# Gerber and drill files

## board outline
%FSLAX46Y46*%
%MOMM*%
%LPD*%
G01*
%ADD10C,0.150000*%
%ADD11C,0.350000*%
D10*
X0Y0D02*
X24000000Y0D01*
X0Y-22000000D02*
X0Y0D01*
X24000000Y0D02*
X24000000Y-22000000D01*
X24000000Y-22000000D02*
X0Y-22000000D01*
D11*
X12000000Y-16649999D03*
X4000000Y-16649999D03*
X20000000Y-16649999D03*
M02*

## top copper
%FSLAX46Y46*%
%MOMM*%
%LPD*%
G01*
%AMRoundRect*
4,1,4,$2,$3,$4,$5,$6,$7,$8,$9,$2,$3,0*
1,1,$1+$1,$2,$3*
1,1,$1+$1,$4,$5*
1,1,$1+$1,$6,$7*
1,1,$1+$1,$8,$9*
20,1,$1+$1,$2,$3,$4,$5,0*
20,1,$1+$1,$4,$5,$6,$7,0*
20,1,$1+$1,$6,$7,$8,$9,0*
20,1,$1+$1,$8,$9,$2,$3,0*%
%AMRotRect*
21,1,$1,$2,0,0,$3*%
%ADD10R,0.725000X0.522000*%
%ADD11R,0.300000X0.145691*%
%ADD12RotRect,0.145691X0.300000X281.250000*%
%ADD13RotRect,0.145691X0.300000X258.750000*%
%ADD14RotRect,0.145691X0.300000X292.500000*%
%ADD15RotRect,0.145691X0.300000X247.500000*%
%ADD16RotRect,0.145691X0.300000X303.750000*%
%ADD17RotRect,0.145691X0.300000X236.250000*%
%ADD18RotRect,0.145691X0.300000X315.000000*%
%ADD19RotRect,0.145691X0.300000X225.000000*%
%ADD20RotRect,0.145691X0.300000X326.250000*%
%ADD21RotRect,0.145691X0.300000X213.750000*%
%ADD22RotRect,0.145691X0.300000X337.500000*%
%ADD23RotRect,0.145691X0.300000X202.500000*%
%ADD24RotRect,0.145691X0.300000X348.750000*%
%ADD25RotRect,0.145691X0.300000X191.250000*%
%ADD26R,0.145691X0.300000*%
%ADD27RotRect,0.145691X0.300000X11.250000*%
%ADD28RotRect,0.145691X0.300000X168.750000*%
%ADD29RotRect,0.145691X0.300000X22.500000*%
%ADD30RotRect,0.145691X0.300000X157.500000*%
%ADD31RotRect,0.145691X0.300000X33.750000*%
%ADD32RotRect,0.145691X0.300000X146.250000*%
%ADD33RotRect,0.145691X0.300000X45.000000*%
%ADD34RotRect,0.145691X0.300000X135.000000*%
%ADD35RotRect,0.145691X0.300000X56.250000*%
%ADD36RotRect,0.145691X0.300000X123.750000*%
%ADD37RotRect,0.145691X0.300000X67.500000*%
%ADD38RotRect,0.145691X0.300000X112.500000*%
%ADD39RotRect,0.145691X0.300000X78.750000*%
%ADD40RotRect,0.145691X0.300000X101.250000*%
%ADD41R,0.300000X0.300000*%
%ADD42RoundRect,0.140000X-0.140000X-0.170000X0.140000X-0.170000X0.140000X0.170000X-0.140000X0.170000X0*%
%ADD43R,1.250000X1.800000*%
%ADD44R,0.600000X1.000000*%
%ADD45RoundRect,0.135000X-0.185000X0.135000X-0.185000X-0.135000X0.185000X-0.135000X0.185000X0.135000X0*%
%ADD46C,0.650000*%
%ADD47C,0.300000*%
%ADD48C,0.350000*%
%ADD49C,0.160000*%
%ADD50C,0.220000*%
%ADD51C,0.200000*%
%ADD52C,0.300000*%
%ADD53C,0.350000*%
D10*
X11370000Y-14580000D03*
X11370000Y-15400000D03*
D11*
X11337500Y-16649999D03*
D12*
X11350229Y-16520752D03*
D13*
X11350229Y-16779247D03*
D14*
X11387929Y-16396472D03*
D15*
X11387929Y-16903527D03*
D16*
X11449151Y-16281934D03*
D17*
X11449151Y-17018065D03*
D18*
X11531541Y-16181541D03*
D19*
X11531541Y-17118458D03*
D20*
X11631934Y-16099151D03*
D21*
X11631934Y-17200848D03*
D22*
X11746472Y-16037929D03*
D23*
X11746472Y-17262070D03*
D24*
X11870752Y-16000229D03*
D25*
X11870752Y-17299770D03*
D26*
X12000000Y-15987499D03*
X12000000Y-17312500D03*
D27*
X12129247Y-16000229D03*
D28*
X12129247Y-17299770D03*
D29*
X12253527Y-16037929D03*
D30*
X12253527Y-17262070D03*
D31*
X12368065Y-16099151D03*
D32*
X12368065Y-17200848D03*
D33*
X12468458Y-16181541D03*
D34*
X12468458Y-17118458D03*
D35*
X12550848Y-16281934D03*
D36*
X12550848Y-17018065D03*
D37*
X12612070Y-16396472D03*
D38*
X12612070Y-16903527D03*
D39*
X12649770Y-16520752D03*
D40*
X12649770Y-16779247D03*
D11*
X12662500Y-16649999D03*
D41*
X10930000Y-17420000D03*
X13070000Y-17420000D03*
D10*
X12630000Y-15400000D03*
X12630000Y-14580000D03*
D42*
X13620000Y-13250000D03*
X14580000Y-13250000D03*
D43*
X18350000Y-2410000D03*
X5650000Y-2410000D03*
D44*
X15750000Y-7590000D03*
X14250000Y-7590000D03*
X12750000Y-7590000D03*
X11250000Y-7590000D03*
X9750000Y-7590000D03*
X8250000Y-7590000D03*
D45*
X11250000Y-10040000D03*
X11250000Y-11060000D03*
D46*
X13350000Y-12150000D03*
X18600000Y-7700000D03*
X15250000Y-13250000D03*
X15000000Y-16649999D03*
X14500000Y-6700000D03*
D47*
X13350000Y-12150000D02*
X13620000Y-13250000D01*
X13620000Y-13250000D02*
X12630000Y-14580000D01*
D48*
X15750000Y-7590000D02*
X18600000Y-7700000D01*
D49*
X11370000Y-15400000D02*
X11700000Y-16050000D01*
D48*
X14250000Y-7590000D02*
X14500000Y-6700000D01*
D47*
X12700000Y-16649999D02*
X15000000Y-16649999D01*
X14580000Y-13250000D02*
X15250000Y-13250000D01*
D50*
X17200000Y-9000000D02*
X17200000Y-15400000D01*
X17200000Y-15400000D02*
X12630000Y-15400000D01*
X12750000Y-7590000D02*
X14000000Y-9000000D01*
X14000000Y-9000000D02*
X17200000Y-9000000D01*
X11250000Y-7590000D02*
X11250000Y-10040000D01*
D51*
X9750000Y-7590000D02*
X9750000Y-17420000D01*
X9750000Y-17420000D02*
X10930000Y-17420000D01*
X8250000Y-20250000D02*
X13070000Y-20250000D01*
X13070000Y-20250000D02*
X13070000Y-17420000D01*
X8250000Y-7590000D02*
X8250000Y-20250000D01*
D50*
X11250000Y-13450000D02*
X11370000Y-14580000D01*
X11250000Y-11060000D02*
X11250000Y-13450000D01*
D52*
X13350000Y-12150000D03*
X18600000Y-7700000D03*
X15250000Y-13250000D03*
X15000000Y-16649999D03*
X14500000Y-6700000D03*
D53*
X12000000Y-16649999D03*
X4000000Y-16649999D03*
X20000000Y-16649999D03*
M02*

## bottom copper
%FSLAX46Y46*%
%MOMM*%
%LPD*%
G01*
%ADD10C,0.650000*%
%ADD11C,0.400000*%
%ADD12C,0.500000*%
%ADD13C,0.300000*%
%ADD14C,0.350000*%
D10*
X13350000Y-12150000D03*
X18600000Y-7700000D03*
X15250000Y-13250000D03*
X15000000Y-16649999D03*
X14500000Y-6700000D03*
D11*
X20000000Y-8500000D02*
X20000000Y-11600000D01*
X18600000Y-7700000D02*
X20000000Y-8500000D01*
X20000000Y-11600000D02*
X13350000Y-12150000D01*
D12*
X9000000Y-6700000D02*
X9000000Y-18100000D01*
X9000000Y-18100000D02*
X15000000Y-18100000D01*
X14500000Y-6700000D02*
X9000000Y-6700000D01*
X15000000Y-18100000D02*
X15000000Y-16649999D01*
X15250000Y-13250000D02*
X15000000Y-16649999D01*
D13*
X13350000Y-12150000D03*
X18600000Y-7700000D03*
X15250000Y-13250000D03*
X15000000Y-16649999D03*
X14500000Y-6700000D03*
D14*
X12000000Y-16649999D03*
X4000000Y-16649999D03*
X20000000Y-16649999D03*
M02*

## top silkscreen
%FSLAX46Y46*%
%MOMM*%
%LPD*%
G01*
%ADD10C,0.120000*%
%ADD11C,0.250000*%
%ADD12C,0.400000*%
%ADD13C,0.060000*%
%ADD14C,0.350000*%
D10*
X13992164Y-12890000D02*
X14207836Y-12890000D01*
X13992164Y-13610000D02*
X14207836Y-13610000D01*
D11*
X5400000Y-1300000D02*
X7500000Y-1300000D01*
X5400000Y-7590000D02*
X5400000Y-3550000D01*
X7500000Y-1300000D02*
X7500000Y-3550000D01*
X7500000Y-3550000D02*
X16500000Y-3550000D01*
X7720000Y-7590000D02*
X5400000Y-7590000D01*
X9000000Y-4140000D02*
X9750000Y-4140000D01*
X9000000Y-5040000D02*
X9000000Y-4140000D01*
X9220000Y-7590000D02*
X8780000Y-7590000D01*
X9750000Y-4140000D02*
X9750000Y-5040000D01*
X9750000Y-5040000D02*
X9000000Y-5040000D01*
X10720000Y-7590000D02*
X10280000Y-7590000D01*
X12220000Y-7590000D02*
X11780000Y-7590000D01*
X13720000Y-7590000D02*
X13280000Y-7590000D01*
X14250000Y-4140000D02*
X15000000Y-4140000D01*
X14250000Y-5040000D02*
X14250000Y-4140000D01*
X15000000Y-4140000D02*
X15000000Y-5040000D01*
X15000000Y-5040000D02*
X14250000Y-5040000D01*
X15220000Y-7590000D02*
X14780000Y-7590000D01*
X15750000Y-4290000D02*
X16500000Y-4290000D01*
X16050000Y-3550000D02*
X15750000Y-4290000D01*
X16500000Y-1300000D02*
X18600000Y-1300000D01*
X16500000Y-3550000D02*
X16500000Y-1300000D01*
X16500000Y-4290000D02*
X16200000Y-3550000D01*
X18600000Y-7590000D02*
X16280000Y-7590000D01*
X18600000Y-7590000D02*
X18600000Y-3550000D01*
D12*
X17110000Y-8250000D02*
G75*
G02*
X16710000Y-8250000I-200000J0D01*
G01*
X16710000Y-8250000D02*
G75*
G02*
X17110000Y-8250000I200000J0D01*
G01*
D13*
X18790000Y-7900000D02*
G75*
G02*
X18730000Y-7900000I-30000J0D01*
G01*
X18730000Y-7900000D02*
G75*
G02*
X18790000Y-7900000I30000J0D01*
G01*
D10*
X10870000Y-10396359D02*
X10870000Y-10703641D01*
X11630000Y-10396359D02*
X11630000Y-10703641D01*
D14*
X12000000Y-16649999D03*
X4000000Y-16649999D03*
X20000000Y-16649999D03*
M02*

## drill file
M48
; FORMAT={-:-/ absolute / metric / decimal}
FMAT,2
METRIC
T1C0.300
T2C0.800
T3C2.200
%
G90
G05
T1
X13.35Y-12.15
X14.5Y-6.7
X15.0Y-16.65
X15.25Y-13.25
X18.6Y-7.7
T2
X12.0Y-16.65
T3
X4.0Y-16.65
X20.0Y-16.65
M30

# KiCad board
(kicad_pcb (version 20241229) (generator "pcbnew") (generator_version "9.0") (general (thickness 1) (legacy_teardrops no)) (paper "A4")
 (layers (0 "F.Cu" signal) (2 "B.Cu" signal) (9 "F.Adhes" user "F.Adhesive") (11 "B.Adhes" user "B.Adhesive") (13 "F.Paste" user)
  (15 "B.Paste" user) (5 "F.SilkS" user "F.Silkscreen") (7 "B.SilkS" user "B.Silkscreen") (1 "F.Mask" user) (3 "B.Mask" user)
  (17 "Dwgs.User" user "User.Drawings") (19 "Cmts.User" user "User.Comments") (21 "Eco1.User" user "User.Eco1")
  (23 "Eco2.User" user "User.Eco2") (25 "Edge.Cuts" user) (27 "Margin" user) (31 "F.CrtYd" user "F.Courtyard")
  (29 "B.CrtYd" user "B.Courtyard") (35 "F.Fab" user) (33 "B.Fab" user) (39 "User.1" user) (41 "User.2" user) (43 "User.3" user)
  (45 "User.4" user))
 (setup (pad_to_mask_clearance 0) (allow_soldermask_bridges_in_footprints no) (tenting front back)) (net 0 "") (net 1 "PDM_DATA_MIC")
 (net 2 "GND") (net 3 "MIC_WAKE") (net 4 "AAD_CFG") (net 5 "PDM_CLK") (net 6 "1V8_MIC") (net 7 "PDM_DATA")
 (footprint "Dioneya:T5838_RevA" (layer "F.Cu") (at 12 16)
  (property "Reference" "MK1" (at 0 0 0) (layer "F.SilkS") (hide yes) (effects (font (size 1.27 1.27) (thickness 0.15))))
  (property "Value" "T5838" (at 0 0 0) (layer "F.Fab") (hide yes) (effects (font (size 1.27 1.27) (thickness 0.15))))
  (pad "" np_thru_hole circle (at 0 0.649999) (size 0.8 0.8) (drill 0.8) (layers "*.Cu" "*.Mask"))
  (pad "1" smd rect (at -0.63 -1.42 90) (size 0.522 0.725) (layers "F.Cu" "F.Mask" "F.Paste") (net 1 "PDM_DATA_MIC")
   (solder_paste_margin -0.05) (thermal_bridge_angle 45))
  (pad "2" smd rect (at -0.63 -0.6 90) (size 0.522 0.725) (layers "F.Cu" "F.Mask" "F.Paste") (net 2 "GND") (solder_paste_margin -0.05)
   (thermal_bridge_angle 45))
  (pad "3" smd rect (at -0.6625 0.649999 270) (size 0.145691 0.3) (layers "F.Cu" "F.Mask") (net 2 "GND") (thermal_bridge_angle 45))
  (pad "3" smd rect (at -0.649771 0.520752 281.25) (size 0.145691 0.3) (layers "F.Cu" "F.Mask") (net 2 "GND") (thermal_bridge_angle 45))
  (pad "3" smd rect (at -0.649771 0.779247 258.75) (size 0.145691 0.3) (layers "F.Cu" "F.Mask") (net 2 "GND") (thermal_bridge_angle 45))
  (pad "3" smd rect (at -0.612071 0.396472 292.5) (size 0.145691 0.3) (layers "F.Cu" "F.Mask") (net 2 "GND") (thermal_bridge_angle 45))
  (pad "3" smd rect (at -0.612071 0.903527 247.5) (size 0.145691 0.3) (layers "F.Cu" "F.Mask") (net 2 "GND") (thermal_bridge_angle 45))
  (pad "3" smd rect (at -0.550849 0.281934 303.75) (size 0.145691 0.3) (layers "F.Cu" "F.Mask") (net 2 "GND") (thermal_bridge_angle 45))
  (pad "3" smd rect (at -0.550849 1.018065 236.25) (size 0.145691 0.3) (layers "F.Cu" "F.Mask") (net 2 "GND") (thermal_bridge_angle 45))
  (pad "3" smd rect (at -0.468459 0.181541 315) (size 0.145691 0.3) (layers "F.Cu" "F.Mask") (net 2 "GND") (thermal_bridge_angle 45))
  (pad "3" smd rect (at -0.468459 1.118458 225) (size 0.145691 0.3) (layers "F.Cu" "F.Mask") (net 2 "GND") (thermal_bridge_angle 45))
  (pad "3" smd rect (at -0.368066 0.099151 326.25) (size 0.145691 0.3) (layers "F.Cu" "F.Mask") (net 2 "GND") (thermal_bridge_angle 45))
  (pad "3" smd rect (at -0.368066 1.200848 213.75) (size 0.145691 0.3) (layers "F.Cu" "F.Mask") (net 2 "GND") (thermal_bridge_angle 45))
  (pad "3" smd rect (at -0.253528 0.037929 337.5) (size 0.145691 0.3) (layers "F.Cu" "F.Mask") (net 2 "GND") (thermal_bridge_angle 45))
  (pad "3" smd rect (at -0.253528 1.26207 202.5) (size 0.145691 0.3) (layers "F.Cu" "F.Mask") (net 2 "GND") (thermal_bridge_angle 45))
  (pad "3" smd rect (at -0.129248 0.000229 348.75) (size 0.145691 0.3) (layers "F.Cu" "F.Mask") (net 2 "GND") (thermal_bridge_angle 45))
  (pad "3" smd rect (at -0.129248 1.29977 191.25) (size 0.145691 0.3) (layers "F.Cu" "F.Mask") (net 2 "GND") (thermal_bridge_angle 45))
  (pad "3" smd rect (at 0 -0.012501) (size 0.145691 0.3) (layers "F.Cu" "F.Mask") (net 2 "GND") (thermal_bridge_angle 45))
  (pad "3" smd rect (at 0 1.3125 180) (size 0.145691 0.3) (layers "F.Cu" "F.Mask") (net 2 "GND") (thermal_bridge_angle 45))
  (pad "3" smd rect (at 0.129247 0.000229 11.25) (size 0.145691 0.3) (layers "F.Cu" "F.Mask") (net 2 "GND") (thermal_bridge_angle 45))
  (pad "3" smd rect (at 0.129247 1.29977 168.75) (size 0.145691 0.3) (layers "F.Cu" "F.Mask") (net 2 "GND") (thermal_bridge_angle 45))
  (pad "3" smd rect (at 0.253527 0.037929 22.5) (size 0.145691 0.3) (layers "F.Cu" "F.Mask") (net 2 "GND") (thermal_bridge_angle 45))
  (pad "3" smd rect (at 0.253527 1.26207 157.5) (size 0.145691 0.3) (layers "F.Cu" "F.Mask") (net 2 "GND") (thermal_bridge_angle 45))
  (pad "3" smd rect (at 0.368065 0.099151 33.75) (size 0.145691 0.3) (layers "F.Cu" "F.Mask") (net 2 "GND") (thermal_bridge_angle 45))
  (pad "3" smd rect (at 0.368065 1.200848 146.25) (size 0.145691 0.3) (layers "F.Cu" "F.Mask") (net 2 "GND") (thermal_bridge_angle 45))
  (pad "3" smd rect (at 0.468458 0.181541 45) (size 0.145691 0.3) (layers "F.Cu" "F.Mask") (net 2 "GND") (thermal_bridge_angle 45))
  (pad "3" smd rect (at 0.468458 1.118458 135) (size 0.145691 0.3) (layers "F.Cu" "F.Mask") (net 2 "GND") (thermal_bridge_angle 45))
  (pad "3" smd rect (at 0.550848 0.281934 56.25) (size 0.145691 0.3) (layers "F.Cu" "F.Mask") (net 2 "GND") (thermal_bridge_angle 45))
  (pad "3" smd rect (at 0.550848 1.018065 123.75) (size 0.145691 0.3) (layers "F.Cu" "F.Mask") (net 2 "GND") (thermal_bridge_angle 45))
  (pad "3" smd rect (at 0.61207 0.396472 67.5) (size 0.145691 0.3) (layers "F.Cu" "F.Mask") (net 2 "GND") (thermal_bridge_angle 45))
  (pad "3" smd rect (at 0.61207 0.903527 112.5) (size 0.145691 0.3) (layers "F.Cu" "F.Mask") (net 2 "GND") (thermal_bridge_angle 45))
  (pad "3" smd rect (at 0.64977 0.520752 78.75) (size 0.145691 0.3) (layers "F.Cu" "F.Mask") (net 2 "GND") (thermal_bridge_angle 45))
  (pad "3" smd rect (at 0.64977 0.779247 101.25) (size 0.145691 0.3) (layers "F.Cu" "F.Mask") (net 2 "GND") (thermal_bridge_angle 45))
  (pad "3" smd rect (at 0.6625 0.649999 90) (size 0.145691 0.3) (layers "F.Cu" "F.Mask") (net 2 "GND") (thermal_bridge_angle 45))
  (pad "4" smd rect (at -1.07 1.42 90) (size 0.3 0.3) (layers "F.Cu" "F.Mask" "F.Paste") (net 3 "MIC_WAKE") (solder_paste_margin -0.015)
   (thermal_bridge_angle 45))
  (pad "5" smd rect (at 1.07 1.42 90) (size 0.3 0.3) (layers "F.Cu" "F.Mask" "F.Paste") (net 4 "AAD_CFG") (solder_paste_margin -0.015)
   (thermal_bridge_angle 45))
  (pad "6" smd rect (at 0.63 -0.6 90) (size 0.522 0.725) (layers "F.Cu" "F.Mask" "F.Paste") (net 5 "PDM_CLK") (solder_paste_margin -0.05)
   (thermal_bridge_angle 45))
  (pad "7" smd rect (at 0.63 -1.42 90) (size 0.522 0.725) (layers "F.Cu" "F.Mask" "F.Paste") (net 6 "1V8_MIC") (solder_paste_margin -0.05)
   (thermal_bridge_angle 45)))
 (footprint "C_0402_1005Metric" (layer "F.Cu") (at 14.1 13.25)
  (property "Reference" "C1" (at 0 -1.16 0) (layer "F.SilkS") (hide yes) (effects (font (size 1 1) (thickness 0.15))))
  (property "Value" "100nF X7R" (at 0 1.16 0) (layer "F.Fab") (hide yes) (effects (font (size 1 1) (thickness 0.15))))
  (fp_line (start -0.107836 -0.36) (end 0.107836 -0.36) (stroke (width 0.12) (type solid)) (layer "F.SilkS"))
  (fp_line (start -0.107836 0.36) (end 0.107836 0.36) (stroke (width 0.12) (type solid)) (layer "F.SilkS"))
  (pad "1" smd roundrect (at -0.48 0) (size 0.56 0.62) (layers "F.Cu" "F.Mask" "F.Paste") (roundrect_rratio 0.25) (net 6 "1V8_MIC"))
  (pad "2" smd roundrect (at 0.48 0) (size 0.56 0.62) (layers "F.Cu" "F.Mask" "F.Paste") (roundrect_rratio 0.25) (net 2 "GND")))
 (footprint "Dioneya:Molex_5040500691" (layer "F.Cu") (at 12 5 180)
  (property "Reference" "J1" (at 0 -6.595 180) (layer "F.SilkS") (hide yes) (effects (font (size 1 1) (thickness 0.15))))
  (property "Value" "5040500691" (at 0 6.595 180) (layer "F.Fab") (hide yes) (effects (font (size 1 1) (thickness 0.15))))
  (fp_line (start 6.6 3.7) (end 4.5 3.7) (stroke (width 0.25) (type solid)) (layer "F.SilkS"))
  (fp_line (start 6.6 -2.59) (end 6.6 1.45) (stroke (width 0.25) (type solid)) (layer "F.SilkS"))
  (fp_line (start 4.5 3.7) (end 4.5 1.45) (stroke (width 0.25) (type solid)) (layer "F.SilkS"))
  (fp_line (start 4.5 1.45) (end -4.5 1.45) (stroke (width 0.25) (type solid)) (layer "F.SilkS"))
  (fp_line (start 4.28 -2.59) (end 6.6 -2.59) (stroke (width 0.25) (type solid)) (layer "F.SilkS"))
  (fp_line (start 3 0.86) (end 2.25 0.86) (stroke (width 0.25) (type solid)) (layer "F.SilkS"))
  (fp_line (start 3 -0.04) (end 3 0.86) (stroke (width 0.25) (type solid)) (layer "F.SilkS"))
  (fp_line (start 2.78 -2.59) (end 3.22 -2.59) (stroke (width 0.25) (type solid)) (layer "F.SilkS"))
  (fp_line (start 2.25 0.86) (end 2.25 -0.04) (stroke (width 0.25) (type solid)) (layer "F.SilkS"))
  (fp_line (start 2.25 -0.04) (end 3 -0.04) (stroke (width 0.25) (type solid)) (layer "F.SilkS"))
  (fp_line (start 1.28 -2.59) (end 1.72 -2.59) (stroke (width 0.25) (type solid)) (layer "F.SilkS"))
  (fp_line (start -0.22 -2.59) (end 0.22 -2.59) (stroke (width 0.25) (type solid)) (layer "F.SilkS"))
  (fp_line (start -1.72 -2.59) (end -1.28 -2.59) (stroke (width 0.25) (type solid)) (layer "F.SilkS"))
  (fp_line (start -2.25 0.86) (end -3 0.86) (stroke (width 0.25) (type solid)) (layer "F.SilkS"))
  (fp_line (start -2.25 -0.04) (end -2.25 0.86) (stroke (width 0.25) (type solid)) (layer "F.SilkS"))
  (fp_line (start -3 0.86) (end -3 -0.04) (stroke (width 0.25) (type solid)) (layer "F.SilkS"))
  (fp_line (start -3 -0.04) (end -2.25 -0.04) (stroke (width 0.25) (type solid)) (layer "F.SilkS"))
  (fp_line (start -3.22 -2.59) (end -2.78 -2.59) (stroke (width 0.25) (type solid)) (layer "F.SilkS"))
  (fp_line (start -3.75 0.71) (end -4.5 0.71) (stroke (width 0.25) (type solid)) (layer "F.SilkS"))
  (fp_line (start -4.05 1.45) (end -3.75 0.71) (stroke (width 0.25) (type solid)) (layer "F.SilkS"))
  (fp_line (start -4.5 3.7) (end -6.6 3.7) (stroke (width 0.25) (type solid)) (layer "F.SilkS"))
  (fp_line (start -4.5 1.45) (end -4.5 3.7) (stroke (width 0.25) (type solid)) (layer "F.SilkS"))
  (fp_line (start -4.5 0.71) (end -4.2 1.45) (stroke (width 0.25) (type solid)) (layer "F.SilkS"))
  (fp_line (start -6.6 -2.59) (end -4.28 -2.59) (stroke (width 0.25) (type solid)) (layer "F.SilkS"))
  (fp_line (start -6.6 -2.59) (end -6.6 1.45) (stroke (width 0.25) (type solid)) (layer "F.SilkS"))
  (fp_circle (center -4.91 -3.25) (end -4.71 -3.25) (stroke (width 0.4) (type solid)) (fill no) (layer "F.SilkS"))
  (fp_circle (center -6.76 -2.9) (end -6.73 -2.9) (stroke (width 0.06) (type solid)) (fill no) (layer "F.SilkS"))
  (pad "" smd rect (at -6.35 2.59) (size 1.25 1.8) (layers "F.Cu" "F.Mask" "F.Paste"))
  (pad "" smd rect (at 6.35 2.59) (size 1.25 1.8) (layers "F.Cu" "F.Mask" "F.Paste"))
  (pad "1" smd rect (at -3.75 -2.59) (size 0.6 1) (layers "F.Cu" "F.Mask" "F.Paste") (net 6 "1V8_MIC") (solder_paste_margin 0))
  (pad "2" smd rect (at -2.25 -2.59) (size 0.6 1) (layers "F.Cu" "F.Mask" "F.Paste") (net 2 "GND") (solder_paste_margin 0))
  (pad "3" smd rect (at -0.75 -2.59) (size 0.6 1) (layers "F.Cu" "F.Mask" "F.Paste") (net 5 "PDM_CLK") (solder_paste_margin 0))
  (pad "4" smd rect (at 0.75 -2.59) (size 0.6 1) (layers "F.Cu" "F.Mask" "F.Paste") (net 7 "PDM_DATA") (solder_paste_margin 0))
  (pad "5" smd rect (at 2.25 -2.59) (size 0.6 1) (layers "F.Cu" "F.Mask" "F.Paste") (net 3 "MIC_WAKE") (solder_paste_margin 0))
  (pad "6" smd rect (at 3.75 -2.59) (size 0.6 1) (layers "F.Cu" "F.Mask" "F.Paste") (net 4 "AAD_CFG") (solder_paste_margin 0)))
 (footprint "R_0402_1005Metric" (layer "F.Cu") (at 11.25 10.55 -90)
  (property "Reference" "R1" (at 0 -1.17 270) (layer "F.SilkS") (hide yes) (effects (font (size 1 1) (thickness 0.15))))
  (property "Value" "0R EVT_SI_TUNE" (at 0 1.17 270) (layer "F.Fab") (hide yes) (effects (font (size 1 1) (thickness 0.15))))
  (fp_line (start -0.153641 0.38) (end 0.153641 0.38) (stroke (width 0.12) (type solid)) (layer "F.SilkS"))
  (fp_line (start -0.153641 -0.38) (end 0.153641 -0.38) (stroke (width 0.12) (type solid)) (layer "F.SilkS"))
  (pad "1" smd roundrect (at -0.51 0 270) (size 0.54 0.64) (layers "F.Cu" "F.Mask" "F.Paste") (roundrect_rratio 0.25) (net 7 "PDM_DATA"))
  (pad "2" smd roundrect (at 0.51 0 270) (size 0.54 0.64) (layers "F.Cu" "F.Mask" "F.Paste") (roundrect_rratio 0.25) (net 1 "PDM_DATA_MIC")))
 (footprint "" (layer "F.Cu") (at 4 16.649999)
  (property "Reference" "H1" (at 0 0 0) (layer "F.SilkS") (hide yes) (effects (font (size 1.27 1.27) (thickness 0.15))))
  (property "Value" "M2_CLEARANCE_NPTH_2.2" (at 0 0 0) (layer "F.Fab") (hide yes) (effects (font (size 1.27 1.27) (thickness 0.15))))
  (pad "" np_thru_hole circle (at 0 0) (size 2.2 2.2) (drill 2.2) (layers "*.Cu" "*.Mask")))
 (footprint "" (layer "F.Cu") (at 20 16.649999)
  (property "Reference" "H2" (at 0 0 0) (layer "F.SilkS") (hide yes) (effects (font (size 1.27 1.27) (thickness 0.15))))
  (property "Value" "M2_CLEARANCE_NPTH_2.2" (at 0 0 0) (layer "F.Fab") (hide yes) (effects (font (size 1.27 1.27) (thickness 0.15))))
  (pad "" np_thru_hole circle (at 0 0) (size 2.2 2.2) (drill 2.2) (layers "*.Cu" "*.Mask")))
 (gr_line (start 0 0) (end 24 0) (stroke (width 0.15) (type default)) (layer "Edge.Cuts"))
 (gr_line (start 0 22) (end 0 0) (stroke (width 0.15) (type default)) (layer "Edge.Cuts"))
 (gr_line (start 24 0) (end 24 22) (stroke (width 0.15) (type default)) (layer "Edge.Cuts"))
 (gr_line (start 24 22) (end 0 22) (stroke (width 0.15) (type default)) (layer "Edge.Cuts"))
 (segment (start 13.35 12.15) (end 13.62 13.25) (width 0.3) (layer "F.Cu") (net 6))
 (segment (start 13.62 13.25) (end 12.63 14.58) (width 0.3) (layer "F.Cu") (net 6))
 (segment (start 15.75 7.59) (end 18.6 7.7) (width 0.35) (layer "F.Cu") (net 6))
 (via (at 13.35 12.15) (size 0.65) (drill 0.3) (layers "F.Cu" "B.Cu") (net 6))
 (via (at 18.6 7.7) (size 0.65) (drill 0.3) (layers "F.Cu" "B.Cu") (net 6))
 (segment (start 20 8.5) (end 20 11.6) (width 0.4) (layer "B.Cu") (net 6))
 (segment (start 18.6 7.7) (end 20 8.5) (width 0.4) (layer "B.Cu") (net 6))
 (segment (start 20 11.6) (end 13.35 12.15) (width 0.4) (layer "B.Cu") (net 6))
 (segment (start 11.37 15.4) (end 11.7 16.05) (width 0.16) (layer "F.Cu") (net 2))
 (segment (start 14.25 7.59) (end 14.5 6.7) (width 0.35) (layer "F.Cu") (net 2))
 (segment (start 12.7 16.649999) (end 15 16.649999) (width 0.3) (layer "F.Cu") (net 2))
 (segment (start 14.58 13.25) (end 15.25 13.25) (width 0.3) (layer "F.Cu") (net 2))
 (via (at 15.25 13.25) (size 0.65) (drill 0.3) (layers "F.Cu" "B.Cu") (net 2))
 (via (at 15 16.649999) (size 0.65) (drill 0.3) (layers "F.Cu" "B.Cu") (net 2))
 (via (at 14.5 6.7) (size 0.65) (drill 0.3) (layers "F.Cu" "B.Cu") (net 2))
 (segment (start 9 6.7) (end 9 18.1) (width 0.5) (layer "B.Cu") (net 2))
 (segment (start 9 18.1) (end 15 18.1) (width 0.5) (layer "B.Cu") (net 2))
 (segment (start 14.5 6.7) (end 9 6.7) (width 0.5) (layer "B.Cu") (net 2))
 (segment (start 15 18.1) (end 15 16.649999) (width 0.5) (layer "B.Cu") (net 2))
 (segment (start 15.25 13.25) (end 15 16.649999) (width 0.5) (layer "B.Cu") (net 2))
 (segment (start 17.2 9) (end 17.2 15.4) (width 0.22) (layer "F.Cu") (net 5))
 (segment (start 17.2 15.4) (end 12.63 15.4) (width 0.22) (layer "F.Cu") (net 5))
 (segment (start 12.75 7.59) (end 14 9) (width 0.22) (layer "F.Cu") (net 5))
 (segment (start 14 9) (end 17.2 9) (width 0.22) (layer "F.Cu") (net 5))
 (segment (start 11.25 7.59) (end 11.25 10.04) (width 0.22) (layer "F.Cu") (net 7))
 (segment (start 9.75 7.59) (end 9.75 17.42) (width 0.2) (layer "F.Cu") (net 3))
 (segment (start 9.75 17.42) (end 10.93 17.42) (width 0.2) (layer "F.Cu") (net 3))
 (segment (start 8.25 20.25) (end 13.07 20.25) (width 0.2) (layer "F.Cu") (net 4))
 (segment (start 13.07 20.25) (end 13.07 17.42) (width 0.2) (layer "F.Cu") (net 4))
 (segment (start 8.25 7.59) (end 8.25 20.25) (width 0.2) (layer "F.Cu") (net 4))
 (segment (start 11.25 13.45) (end 11.37 14.58) (width 0.22) (layer "F.Cu") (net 1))
 (segment (start 11.25 11.06) (end 11.25 13.45) (width 0.22) (layer "F.Cu") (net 1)))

